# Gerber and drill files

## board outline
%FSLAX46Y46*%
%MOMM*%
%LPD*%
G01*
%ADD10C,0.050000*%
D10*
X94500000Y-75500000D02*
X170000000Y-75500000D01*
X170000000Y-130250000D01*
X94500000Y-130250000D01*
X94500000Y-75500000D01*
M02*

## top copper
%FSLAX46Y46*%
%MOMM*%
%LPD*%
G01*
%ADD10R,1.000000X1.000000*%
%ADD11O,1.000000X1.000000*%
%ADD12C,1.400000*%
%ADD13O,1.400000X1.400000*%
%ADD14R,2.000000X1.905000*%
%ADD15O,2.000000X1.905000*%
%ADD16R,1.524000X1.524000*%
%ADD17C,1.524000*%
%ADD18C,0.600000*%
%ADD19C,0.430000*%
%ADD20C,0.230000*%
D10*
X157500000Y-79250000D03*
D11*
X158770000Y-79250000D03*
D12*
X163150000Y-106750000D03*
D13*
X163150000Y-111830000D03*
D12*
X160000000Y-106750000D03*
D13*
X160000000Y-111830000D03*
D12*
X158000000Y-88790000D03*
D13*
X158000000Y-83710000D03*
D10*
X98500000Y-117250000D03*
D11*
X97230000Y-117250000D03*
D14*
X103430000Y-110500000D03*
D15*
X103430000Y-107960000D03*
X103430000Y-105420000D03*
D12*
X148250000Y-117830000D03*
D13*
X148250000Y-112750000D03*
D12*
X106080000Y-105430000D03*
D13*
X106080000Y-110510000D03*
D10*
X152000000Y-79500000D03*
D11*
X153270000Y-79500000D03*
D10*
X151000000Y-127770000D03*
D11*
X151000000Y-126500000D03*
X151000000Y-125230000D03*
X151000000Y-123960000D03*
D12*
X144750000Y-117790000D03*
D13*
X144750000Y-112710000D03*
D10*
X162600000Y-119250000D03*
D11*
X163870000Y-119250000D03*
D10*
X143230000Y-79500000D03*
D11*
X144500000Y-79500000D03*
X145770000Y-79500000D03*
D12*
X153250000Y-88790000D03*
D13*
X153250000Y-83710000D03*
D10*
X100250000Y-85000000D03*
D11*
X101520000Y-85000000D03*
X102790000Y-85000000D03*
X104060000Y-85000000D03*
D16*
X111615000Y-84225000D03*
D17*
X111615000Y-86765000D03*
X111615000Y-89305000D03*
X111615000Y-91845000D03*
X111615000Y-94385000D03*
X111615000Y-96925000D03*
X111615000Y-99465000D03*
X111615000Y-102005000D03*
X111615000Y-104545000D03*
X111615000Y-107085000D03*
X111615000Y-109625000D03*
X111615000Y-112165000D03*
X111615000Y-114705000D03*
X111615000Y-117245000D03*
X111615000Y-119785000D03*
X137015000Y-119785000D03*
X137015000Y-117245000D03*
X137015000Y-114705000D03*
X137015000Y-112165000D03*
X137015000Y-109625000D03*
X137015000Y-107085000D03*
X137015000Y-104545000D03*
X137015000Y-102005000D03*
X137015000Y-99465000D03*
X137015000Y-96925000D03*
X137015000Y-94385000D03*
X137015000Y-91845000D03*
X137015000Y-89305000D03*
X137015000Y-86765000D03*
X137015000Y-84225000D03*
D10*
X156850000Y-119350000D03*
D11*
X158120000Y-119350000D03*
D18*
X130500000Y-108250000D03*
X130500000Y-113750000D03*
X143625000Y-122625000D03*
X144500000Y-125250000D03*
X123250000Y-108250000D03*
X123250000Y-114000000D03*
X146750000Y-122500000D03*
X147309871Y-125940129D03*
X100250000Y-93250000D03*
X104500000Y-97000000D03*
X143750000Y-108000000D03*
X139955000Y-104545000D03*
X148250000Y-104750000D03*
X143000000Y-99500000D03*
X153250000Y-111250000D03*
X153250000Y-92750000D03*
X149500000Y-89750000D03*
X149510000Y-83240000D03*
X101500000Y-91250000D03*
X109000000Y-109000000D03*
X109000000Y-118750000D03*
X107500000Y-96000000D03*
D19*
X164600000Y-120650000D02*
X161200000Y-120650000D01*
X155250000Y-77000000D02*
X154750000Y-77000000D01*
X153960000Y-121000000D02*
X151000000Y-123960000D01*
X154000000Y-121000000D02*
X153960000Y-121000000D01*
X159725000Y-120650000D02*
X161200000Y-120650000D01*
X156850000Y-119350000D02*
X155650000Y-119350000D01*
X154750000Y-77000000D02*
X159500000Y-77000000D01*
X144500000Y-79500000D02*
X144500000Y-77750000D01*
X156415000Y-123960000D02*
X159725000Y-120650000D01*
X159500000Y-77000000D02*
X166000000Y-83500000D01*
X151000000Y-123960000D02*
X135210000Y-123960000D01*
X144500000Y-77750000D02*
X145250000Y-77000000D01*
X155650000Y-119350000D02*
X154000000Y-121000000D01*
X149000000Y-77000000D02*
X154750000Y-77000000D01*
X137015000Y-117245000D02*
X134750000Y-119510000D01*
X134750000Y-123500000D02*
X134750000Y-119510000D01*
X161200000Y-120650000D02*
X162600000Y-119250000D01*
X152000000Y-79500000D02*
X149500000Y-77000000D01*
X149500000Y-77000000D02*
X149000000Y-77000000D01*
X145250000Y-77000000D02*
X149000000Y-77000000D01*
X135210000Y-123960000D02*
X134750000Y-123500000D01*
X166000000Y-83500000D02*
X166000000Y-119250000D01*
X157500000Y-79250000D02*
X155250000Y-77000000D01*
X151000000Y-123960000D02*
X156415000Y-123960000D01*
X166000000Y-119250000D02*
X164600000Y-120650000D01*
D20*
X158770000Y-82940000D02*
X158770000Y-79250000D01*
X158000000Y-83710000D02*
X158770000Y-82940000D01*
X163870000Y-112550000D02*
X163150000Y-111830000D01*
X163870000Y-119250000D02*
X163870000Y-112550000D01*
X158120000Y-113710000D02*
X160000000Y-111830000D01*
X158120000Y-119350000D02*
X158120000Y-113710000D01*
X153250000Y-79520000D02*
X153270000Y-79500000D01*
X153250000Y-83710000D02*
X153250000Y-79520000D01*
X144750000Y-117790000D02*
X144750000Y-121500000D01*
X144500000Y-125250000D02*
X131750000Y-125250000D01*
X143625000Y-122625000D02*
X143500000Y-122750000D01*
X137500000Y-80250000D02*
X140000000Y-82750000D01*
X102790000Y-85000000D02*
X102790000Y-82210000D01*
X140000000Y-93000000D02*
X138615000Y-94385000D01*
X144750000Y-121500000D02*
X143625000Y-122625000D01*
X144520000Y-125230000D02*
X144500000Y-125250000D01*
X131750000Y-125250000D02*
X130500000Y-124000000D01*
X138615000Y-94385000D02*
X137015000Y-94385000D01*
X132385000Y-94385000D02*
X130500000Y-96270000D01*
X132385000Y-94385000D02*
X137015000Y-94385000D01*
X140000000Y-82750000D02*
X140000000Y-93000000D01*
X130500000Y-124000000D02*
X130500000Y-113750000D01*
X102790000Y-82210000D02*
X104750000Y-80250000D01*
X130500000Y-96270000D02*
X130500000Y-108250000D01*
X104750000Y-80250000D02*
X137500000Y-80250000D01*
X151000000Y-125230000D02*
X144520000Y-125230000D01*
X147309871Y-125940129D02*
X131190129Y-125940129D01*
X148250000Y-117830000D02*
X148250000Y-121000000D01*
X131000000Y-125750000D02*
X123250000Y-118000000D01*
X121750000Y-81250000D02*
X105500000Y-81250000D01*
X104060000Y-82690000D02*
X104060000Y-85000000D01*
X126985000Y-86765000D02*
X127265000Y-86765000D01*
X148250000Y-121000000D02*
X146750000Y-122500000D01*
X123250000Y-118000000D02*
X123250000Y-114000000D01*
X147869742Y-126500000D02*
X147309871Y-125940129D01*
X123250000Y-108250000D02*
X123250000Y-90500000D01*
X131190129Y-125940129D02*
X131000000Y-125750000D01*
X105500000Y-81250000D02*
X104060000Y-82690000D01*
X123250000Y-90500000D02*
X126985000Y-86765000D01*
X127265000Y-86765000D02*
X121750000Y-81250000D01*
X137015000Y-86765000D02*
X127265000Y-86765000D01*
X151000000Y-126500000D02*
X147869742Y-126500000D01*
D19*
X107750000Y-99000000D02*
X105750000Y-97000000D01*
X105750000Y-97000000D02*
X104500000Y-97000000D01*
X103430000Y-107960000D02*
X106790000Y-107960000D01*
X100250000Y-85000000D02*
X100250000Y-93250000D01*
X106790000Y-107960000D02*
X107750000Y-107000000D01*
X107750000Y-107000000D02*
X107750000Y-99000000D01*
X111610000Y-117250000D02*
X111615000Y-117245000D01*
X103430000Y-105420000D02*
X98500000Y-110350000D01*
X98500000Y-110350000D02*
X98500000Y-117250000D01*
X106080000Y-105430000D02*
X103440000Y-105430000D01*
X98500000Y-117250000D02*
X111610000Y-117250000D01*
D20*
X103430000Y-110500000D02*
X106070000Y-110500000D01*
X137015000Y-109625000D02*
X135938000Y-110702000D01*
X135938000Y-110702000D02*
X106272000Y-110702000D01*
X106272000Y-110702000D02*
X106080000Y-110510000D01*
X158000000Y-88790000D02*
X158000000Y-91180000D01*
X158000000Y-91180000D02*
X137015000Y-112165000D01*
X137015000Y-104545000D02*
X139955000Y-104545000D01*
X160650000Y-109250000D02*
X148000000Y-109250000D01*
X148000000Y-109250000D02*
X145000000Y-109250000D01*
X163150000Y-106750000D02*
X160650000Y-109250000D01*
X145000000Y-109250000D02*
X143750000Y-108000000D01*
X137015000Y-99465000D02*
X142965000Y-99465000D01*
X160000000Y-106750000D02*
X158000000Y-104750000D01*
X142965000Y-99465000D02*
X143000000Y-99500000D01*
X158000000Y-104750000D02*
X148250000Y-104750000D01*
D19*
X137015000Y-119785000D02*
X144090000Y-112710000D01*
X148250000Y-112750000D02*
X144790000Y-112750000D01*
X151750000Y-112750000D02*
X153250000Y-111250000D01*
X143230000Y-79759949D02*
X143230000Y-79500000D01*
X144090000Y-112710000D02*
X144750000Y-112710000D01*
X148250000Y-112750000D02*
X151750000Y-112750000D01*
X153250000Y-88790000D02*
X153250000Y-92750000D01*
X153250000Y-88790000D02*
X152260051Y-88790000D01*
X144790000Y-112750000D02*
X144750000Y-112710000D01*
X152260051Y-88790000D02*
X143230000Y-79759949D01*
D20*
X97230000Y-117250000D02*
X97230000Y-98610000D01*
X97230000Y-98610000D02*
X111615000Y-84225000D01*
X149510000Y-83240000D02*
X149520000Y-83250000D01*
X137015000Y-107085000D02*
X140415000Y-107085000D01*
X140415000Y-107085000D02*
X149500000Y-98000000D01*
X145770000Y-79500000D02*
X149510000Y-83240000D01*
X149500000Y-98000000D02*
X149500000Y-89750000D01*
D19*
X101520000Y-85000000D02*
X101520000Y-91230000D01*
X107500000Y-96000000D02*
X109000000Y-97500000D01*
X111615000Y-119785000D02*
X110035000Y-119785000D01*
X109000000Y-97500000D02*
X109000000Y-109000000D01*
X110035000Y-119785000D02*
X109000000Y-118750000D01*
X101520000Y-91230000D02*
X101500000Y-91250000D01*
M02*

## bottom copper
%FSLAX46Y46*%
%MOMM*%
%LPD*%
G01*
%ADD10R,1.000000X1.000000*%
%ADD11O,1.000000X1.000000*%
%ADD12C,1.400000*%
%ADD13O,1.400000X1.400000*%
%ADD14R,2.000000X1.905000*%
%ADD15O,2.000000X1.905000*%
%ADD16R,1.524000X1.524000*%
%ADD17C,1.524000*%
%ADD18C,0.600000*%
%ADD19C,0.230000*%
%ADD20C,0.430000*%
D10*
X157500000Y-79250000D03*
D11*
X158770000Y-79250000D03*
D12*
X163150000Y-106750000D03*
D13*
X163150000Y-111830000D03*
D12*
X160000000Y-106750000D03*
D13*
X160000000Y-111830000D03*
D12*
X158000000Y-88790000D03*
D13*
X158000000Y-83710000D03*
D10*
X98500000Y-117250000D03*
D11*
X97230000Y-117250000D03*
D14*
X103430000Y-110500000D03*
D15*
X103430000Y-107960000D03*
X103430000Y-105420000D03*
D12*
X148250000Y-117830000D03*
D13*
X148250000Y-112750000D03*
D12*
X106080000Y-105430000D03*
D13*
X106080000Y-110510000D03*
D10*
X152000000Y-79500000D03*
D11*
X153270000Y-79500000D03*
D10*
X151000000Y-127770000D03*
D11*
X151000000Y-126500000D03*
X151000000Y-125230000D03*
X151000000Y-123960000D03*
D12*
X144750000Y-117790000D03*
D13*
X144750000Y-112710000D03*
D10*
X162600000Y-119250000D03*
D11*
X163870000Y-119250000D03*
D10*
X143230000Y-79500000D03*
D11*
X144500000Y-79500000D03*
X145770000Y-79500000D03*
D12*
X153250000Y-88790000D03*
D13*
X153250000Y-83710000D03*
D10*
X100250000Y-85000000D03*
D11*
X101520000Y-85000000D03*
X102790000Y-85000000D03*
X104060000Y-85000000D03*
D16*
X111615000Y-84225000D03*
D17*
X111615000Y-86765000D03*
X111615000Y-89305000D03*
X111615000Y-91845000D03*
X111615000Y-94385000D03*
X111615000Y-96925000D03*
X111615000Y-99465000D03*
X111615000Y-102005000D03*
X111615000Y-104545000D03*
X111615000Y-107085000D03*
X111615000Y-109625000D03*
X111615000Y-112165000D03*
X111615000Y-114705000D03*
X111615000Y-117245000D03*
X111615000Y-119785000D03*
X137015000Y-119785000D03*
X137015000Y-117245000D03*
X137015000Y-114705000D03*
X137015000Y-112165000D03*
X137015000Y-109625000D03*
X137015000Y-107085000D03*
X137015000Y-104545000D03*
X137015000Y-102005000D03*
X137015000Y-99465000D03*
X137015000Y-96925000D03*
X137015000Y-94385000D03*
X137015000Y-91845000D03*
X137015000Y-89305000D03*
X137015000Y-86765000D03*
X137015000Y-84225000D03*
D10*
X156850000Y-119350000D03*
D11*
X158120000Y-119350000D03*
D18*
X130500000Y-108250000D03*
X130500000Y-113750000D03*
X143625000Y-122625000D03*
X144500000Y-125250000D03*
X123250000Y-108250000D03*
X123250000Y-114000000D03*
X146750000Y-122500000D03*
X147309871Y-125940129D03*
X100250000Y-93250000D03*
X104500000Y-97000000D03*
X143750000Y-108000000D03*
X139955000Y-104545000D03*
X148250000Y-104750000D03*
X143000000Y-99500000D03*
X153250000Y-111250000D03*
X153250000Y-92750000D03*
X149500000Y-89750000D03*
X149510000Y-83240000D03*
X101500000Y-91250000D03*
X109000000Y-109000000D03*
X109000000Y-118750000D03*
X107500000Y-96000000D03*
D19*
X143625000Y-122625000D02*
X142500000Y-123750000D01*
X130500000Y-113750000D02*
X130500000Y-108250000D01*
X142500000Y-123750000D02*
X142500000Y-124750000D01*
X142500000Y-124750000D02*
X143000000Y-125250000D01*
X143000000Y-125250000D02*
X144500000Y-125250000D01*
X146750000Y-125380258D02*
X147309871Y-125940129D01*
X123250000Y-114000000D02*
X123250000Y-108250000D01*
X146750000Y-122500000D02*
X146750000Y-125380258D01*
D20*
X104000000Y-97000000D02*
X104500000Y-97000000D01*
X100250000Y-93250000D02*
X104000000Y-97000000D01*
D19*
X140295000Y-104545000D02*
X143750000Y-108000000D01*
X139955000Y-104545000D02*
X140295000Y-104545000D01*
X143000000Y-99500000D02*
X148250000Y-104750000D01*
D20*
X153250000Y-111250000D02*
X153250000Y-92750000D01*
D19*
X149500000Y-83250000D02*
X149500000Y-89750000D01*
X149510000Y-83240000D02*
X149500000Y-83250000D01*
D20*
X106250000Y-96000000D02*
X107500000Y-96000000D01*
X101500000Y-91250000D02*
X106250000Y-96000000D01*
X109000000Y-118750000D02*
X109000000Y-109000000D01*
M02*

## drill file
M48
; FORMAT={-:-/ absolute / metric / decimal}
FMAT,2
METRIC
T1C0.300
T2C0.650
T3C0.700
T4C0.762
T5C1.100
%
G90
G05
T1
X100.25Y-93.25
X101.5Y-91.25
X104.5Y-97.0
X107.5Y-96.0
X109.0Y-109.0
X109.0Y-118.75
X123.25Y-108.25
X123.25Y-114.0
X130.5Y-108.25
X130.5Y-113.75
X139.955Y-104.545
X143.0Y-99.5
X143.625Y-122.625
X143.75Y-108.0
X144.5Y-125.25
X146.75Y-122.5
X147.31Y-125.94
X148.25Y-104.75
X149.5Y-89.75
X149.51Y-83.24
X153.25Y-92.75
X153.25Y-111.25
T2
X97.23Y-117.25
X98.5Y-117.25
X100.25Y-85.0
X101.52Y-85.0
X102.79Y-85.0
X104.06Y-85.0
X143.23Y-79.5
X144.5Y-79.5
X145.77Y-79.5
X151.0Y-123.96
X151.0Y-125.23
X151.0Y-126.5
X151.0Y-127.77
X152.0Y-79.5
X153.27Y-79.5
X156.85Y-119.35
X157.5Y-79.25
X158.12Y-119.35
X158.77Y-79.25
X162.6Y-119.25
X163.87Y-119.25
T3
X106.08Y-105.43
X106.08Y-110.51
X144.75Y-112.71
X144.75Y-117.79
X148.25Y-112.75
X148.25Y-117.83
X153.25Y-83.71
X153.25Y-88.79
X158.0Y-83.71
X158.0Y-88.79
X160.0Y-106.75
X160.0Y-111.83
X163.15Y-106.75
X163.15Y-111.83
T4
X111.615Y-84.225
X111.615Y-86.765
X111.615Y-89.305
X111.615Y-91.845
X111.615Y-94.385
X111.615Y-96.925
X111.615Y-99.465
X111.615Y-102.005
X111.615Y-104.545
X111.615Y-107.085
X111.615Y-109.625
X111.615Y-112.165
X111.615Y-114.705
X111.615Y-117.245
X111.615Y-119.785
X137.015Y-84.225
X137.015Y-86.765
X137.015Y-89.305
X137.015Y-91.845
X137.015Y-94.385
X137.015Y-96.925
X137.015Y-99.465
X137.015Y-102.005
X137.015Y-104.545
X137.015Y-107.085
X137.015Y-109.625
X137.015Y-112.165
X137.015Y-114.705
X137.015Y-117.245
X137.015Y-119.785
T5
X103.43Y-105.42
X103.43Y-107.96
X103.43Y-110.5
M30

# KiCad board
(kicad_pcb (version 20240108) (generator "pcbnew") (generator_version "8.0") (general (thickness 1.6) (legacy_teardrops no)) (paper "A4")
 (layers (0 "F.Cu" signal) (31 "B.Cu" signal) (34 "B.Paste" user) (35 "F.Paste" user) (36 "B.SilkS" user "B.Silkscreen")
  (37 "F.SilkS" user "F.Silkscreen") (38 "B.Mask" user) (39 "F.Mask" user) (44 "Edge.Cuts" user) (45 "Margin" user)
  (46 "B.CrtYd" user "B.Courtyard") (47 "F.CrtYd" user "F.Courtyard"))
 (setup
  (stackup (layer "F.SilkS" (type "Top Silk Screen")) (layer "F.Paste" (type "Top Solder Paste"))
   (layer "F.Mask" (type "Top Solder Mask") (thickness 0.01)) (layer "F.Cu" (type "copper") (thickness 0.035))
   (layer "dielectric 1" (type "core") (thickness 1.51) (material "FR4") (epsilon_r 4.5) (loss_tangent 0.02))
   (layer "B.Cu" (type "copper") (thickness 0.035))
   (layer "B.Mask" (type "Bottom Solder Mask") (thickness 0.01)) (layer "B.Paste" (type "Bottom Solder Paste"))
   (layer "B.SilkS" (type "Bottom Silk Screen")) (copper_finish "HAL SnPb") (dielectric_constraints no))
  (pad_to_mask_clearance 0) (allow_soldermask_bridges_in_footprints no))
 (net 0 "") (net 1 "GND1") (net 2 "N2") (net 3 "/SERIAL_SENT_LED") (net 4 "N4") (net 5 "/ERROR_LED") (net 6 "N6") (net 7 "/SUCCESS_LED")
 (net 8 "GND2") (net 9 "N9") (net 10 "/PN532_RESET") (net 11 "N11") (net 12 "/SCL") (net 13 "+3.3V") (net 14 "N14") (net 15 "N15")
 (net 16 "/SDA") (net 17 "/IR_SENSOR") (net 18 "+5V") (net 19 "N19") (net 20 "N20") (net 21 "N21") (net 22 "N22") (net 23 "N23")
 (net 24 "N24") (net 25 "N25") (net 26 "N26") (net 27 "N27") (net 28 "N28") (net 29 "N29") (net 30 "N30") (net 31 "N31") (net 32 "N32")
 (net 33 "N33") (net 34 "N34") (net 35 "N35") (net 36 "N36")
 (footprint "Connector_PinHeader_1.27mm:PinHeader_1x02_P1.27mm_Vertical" (layer "F.Cu") (at 157.5 79.25 90)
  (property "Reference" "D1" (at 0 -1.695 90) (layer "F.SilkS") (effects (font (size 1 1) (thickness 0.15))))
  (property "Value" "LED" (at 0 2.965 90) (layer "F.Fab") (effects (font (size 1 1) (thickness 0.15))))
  (pad "1" thru_hole rect (at 0 0 90) (size 1 1) (drill 0.65) (layers "*.Cu" "*.Mask") (remove_unused_layers no) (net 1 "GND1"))
  (pad "2" thru_hole oval (at 0 1.27 90) (size 1 1) (drill 0.65) (layers "*.Cu" "*.Mask") (remove_unused_layers no) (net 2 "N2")))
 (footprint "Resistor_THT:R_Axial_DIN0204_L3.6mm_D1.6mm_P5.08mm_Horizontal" (layer "F.Cu") (at 163.15 106.75 -90)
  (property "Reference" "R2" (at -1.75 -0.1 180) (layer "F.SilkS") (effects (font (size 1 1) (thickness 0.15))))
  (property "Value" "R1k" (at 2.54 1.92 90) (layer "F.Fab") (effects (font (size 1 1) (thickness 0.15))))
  (pad "1" thru_hole circle (at 0 0 270) (size 1.4 1.4) (drill 0.7) (layers "*.Cu" "*.Mask") (remove_unused_layers no)
   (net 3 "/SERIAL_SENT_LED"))
  (pad "2" thru_hole oval (at 5.08 0 270) (size 1.4 1.4) (drill 0.7) (layers "*.Cu" "*.Mask") (remove_unused_layers no) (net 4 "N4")))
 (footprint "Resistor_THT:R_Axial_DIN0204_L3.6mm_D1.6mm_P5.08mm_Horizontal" (layer "F.Cu") (at 160 106.75 -90)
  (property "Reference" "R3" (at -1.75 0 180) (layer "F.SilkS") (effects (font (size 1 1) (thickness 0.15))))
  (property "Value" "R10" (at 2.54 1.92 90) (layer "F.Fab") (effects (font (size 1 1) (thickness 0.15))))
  (pad "1" thru_hole circle (at 0 0 270) (size 1.4 1.4) (drill 0.7) (layers "*.Cu" "*.Mask") (remove_unused_layers no) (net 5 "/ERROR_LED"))
  (pad "2" thru_hole oval (at 5.08 0 270) (size 1.4 1.4) (drill 0.7) (layers "*.Cu" "*.Mask") (remove_unused_layers no) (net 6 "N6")))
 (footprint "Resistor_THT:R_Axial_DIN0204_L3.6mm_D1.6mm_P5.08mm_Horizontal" (layer "F.Cu") (at 158 88.79 90)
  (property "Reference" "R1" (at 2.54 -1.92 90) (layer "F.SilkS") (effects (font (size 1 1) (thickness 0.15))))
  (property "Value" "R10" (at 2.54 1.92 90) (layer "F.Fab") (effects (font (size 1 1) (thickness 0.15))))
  (pad "1" thru_hole circle (at 0 0 90) (size 1.4 1.4) (drill 0.7) (layers "*.Cu" "*.Mask") (remove_unused_layers no) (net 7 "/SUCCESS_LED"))
  (pad "2" thru_hole oval (at 5.08 0 90) (size 1.4 1.4) (drill 0.7) (layers "*.Cu" "*.Mask") (remove_unused_layers no) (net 2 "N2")))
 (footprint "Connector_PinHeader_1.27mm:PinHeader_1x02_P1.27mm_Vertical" (layer "F.Cu") (at 98.5 117.25 -90)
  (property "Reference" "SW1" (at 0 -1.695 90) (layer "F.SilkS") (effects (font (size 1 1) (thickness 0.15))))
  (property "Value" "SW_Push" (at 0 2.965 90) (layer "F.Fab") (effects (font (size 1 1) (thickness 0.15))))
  (pad "1" thru_hole rect (at 0 0 270) (size 1 1) (drill 0.65) (layers "*.Cu" "*.Mask") (remove_unused_layers no) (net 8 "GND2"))
  (pad "2" thru_hole oval (at 0 1.27 270) (size 1 1) (drill 0.65) (layers "*.Cu" "*.Mask") (remove_unused_layers no) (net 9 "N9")))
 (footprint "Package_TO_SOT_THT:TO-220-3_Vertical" (layer "F.Cu") (at 103.43 110.5 90)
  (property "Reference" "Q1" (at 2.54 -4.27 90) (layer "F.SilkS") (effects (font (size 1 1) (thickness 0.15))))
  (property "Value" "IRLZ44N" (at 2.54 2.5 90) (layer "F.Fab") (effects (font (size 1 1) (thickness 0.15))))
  (pad "1" thru_hole rect (at 0 0 90) (size 1.905 2) (drill 1.1) (layers "*.Cu" "*.Mask") (remove_unused_layers no) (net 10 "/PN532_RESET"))
  (pad "2" thru_hole oval (at 2.54 0 90) (size 1.905 2) (drill 1.1) (layers "*.Cu" "*.Mask") (remove_unused_layers no) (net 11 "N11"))
  (pad "3" thru_hole oval (at 5.08 0 90) (size 1.905 2) (drill 1.1) (layers "*.Cu" "*.Mask") (remove_unused_layers no) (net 8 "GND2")))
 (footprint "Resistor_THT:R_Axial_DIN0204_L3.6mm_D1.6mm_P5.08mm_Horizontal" (layer "F.Cu") (at 148.25 117.83 90)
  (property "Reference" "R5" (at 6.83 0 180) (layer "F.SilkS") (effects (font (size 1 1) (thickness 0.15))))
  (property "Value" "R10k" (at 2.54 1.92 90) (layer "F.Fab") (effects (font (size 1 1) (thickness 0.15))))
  (pad "1" thru_hole circle (at 0 0 90) (size 1.4 1.4) (drill 0.7) (layers "*.Cu" "*.Mask") (remove_unused_layers no) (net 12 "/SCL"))
  (pad "2" thru_hole oval (at 5.08 0 90) (size 1.4 1.4) (drill 0.7) (layers "*.Cu" "*.Mask") (remove_unused_layers no) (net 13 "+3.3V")))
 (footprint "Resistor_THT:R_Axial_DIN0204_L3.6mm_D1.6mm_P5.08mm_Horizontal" (layer "F.Cu") (at 106.08 105.43 -90)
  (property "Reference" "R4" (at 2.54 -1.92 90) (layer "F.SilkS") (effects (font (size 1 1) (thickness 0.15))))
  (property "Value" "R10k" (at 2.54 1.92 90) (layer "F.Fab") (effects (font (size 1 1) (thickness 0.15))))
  (pad "1" thru_hole circle (at 0 0 270) (size 1.4 1.4) (drill 0.7) (layers "*.Cu" "*.Mask") (remove_unused_layers no) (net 8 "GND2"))
  (pad "2" thru_hole oval (at 5.08 0 270) (size 1.4 1.4) (drill 0.7) (layers "*.Cu" "*.Mask") (remove_unused_layers no)
   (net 10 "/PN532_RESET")))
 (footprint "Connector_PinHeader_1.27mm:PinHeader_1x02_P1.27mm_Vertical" (layer "F.Cu") (at 152 79.5 90)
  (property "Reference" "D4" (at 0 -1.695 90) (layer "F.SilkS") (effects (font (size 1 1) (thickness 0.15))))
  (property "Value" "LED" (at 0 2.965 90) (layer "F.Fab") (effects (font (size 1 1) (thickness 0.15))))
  (pad "1" thru_hole rect (at 0 0 90) (size 1 1) (drill 0.65) (layers "*.Cu" "*.Mask") (remove_unused_layers no) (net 1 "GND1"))
  (pad "2" thru_hole oval (at 0 1.27 90) (size 1 1) (drill 0.65) (layers "*.Cu" "*.Mask") (remove_unused_layers no) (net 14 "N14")))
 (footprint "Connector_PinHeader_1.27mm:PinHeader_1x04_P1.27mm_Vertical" (layer "F.Cu") (at 151 127.77 180)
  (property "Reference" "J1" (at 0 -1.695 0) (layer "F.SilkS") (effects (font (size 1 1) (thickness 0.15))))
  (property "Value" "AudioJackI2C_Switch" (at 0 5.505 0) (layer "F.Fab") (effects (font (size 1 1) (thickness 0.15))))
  (pad "1" thru_hole rect (at 0 0 180) (size 1 1) (drill 0.65) (layers "*.Cu" "*.Mask") (remove_unused_layers no) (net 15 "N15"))
  (pad "2" thru_hole oval (at 0 1.27 180) (size 1 1) (drill 0.65) (layers "*.Cu" "*.Mask") (remove_unused_layers no) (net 12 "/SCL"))
  (pad "3" thru_hole oval (at 0 2.54 180) (size 1 1) (drill 0.65) (layers "*.Cu" "*.Mask") (remove_unused_layers no) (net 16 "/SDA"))
  (pad "4" thru_hole oval (at 0 3.81 180) (size 1 1) (drill 0.65) (layers "*.Cu" "*.Mask") (remove_unused_layers no) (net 1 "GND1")))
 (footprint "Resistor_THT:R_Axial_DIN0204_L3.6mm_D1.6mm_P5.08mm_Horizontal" (layer "F.Cu") (at 144.75 117.79 90)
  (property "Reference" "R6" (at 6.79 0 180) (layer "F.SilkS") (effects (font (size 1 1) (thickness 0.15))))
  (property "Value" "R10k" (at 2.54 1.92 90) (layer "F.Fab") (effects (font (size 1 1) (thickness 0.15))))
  (pad "1" thru_hole circle (at 0 0 90) (size 1.4 1.4) (drill 0.7) (layers "*.Cu" "*.Mask") (remove_unused_layers no) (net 16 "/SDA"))
  (pad "2" thru_hole oval (at 5.08 0 90) (size 1.4 1.4) (drill 0.7) (layers "*.Cu" "*.Mask") (remove_unused_layers no) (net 13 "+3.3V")))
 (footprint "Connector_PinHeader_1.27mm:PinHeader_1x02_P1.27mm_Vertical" (layer "F.Cu") (at 162.6 119.25 90)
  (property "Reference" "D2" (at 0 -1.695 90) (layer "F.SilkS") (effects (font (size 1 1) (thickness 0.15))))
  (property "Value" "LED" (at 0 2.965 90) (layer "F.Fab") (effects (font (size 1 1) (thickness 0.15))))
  (pad "1" thru_hole rect (at 0 0 90) (size 1 1) (drill 0.65) (layers "*.Cu" "*.Mask") (remove_unused_layers no) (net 1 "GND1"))
  (pad "2" thru_hole oval (at 0 1.27 90) (size 1 1) (drill 0.65) (layers "*.Cu" "*.Mask") (remove_unused_layers no) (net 4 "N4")))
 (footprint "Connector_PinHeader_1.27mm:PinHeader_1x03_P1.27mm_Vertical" (layer "F.Cu") (at 143.23 79.5 90)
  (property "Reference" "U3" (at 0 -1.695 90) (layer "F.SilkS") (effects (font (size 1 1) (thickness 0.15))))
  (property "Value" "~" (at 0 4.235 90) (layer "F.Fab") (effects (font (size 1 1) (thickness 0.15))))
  (pad "1" thru_hole rect (at 0 0 90) (size 1 1) (drill 0.65) (layers "*.Cu" "*.Mask") (remove_unused_layers no) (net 13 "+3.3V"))
  (pad "2" thru_hole oval (at 0 1.27 90) (size 1 1) (drill 0.65) (layers "*.Cu" "*.Mask") (remove_unused_layers no) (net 1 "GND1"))
  (pad "3" thru_hole oval (at 0 2.54 90) (size 1 1) (drill 0.65) (layers "*.Cu" "*.Mask") (remove_unused_layers no) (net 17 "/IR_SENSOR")))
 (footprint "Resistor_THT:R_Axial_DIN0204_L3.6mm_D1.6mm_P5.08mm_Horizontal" (layer "F.Cu") (at 153.25 88.79 90)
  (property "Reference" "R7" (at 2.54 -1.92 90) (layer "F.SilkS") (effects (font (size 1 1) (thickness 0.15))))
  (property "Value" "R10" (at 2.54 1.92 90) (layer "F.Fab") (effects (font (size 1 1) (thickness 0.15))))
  (pad "1" thru_hole circle (at 0 0 90) (size 1.4 1.4) (drill 0.7) (layers "*.Cu" "*.Mask") (remove_unused_layers no) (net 13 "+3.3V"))
  (pad "2" thru_hole oval (at 5.08 0 90) (size 1.4 1.4) (drill 0.7) (layers "*.Cu" "*.Mask") (remove_unused_layers no) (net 14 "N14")))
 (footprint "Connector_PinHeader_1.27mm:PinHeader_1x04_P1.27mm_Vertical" (layer "F.Cu") (at 100.25 85 90)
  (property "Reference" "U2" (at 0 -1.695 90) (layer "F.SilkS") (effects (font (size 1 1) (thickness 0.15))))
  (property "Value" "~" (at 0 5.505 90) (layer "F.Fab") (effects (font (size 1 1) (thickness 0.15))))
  (pad "1" thru_hole rect (at 0 0 90) (size 1 1) (drill 0.65) (layers "*.Cu" "*.Mask") (remove_unused_layers no) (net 11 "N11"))
  (pad "2" thru_hole oval (at 0 1.27 90) (size 1 1) (drill 0.65) (layers "*.Cu" "*.Mask") (remove_unused_layers no) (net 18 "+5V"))
  (pad "3" thru_hole oval (at 0 2.54 90) (size 1 1) (drill 0.65) (layers "*.Cu" "*.Mask") (remove_unused_layers no) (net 16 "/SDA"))
  (pad "4" thru_hole oval (at 0 3.81 90) (size 1 1) (drill 0.65) (layers "*.Cu" "*.Mask") (remove_unused_layers no) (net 12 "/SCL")))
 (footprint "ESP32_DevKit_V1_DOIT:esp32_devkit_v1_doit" (layer "F.Cu") (at 124.315 84.225)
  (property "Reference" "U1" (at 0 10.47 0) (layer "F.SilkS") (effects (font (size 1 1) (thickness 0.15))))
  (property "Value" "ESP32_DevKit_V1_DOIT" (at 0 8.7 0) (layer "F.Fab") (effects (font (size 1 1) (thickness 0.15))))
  (pad "1" thru_hole rect (at -12.7 0) (size 1.524 1.524) (drill 0.762) (layers "*.Cu" "*.Mask") (remove_unused_layers no) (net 9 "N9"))
  (pad "2" thru_hole circle (at -12.7 2.54) (size 1.524 1.524) (drill 0.762) (layers "*.Cu" "*.Mask") (remove_unused_layers no)
   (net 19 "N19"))
  (pad "3" thru_hole circle (at -12.7 5.08) (size 1.524 1.524) (drill 0.762) (layers "*.Cu" "*.Mask") (remove_unused_layers no)
   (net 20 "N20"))
  (pad "4" thru_hole circle (at -12.7 7.62) (size 1.524 1.524) (drill 0.762) (layers "*.Cu" "*.Mask") (remove_unused_layers no)
   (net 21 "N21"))
  (pad "5" thru_hole circle (at -12.7 10.16) (size 1.524 1.524) (drill 0.762) (layers "*.Cu" "*.Mask") (remove_unused_layers no)
   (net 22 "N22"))
  (pad "6" thru_hole circle (at -12.7 12.7) (size 1.524 1.524) (drill 0.762) (layers "*.Cu" "*.Mask") (remove_unused_layers no)
   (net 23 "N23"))
  (pad "7" thru_hole circle (at -12.7 15.24) (size 1.524 1.524) (drill 0.762) (layers "*.Cu" "*.Mask") (remove_unused_layers no)
   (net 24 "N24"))
  (pad "8" thru_hole circle (at -12.7 17.78) (size 1.524 1.524) (drill 0.762) (layers "*.Cu" "*.Mask") (remove_unused_layers no)
   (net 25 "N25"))
  (pad "9" thru_hole circle (at -12.7 20.32) (size 1.524 1.524) (drill 0.762) (layers "*.Cu" "*.Mask") (remove_unused_layers no)
   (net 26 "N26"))
  (pad "10" thru_hole circle (at -12.7 22.86) (size 1.524 1.524) (drill 0.762) (layers "*.Cu" "*.Mask") (remove_unused_layers no)
   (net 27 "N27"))
  (pad "11" thru_hole circle (at -12.7 25.4) (size 1.524 1.524) (drill 0.762) (layers "*.Cu" "*.Mask") (remove_unused_layers no)
   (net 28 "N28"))
  (pad "12" thru_hole circle (at -12.7 27.94) (size 1.524 1.524) (drill 0.762) (layers "*.Cu" "*.Mask") (remove_unused_layers no)
   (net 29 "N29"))
  (pad "13" thru_hole circle (at -12.7 30.48) (size 1.524 1.524) (drill 0.762) (layers "*.Cu" "*.Mask") (remove_unused_layers no)
   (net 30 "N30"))
  (pad "14" thru_hole circle (at -12.7 33.02) (size 1.524 1.524) (drill 0.762) (layers "*.Cu" "*.Mask") (remove_unused_layers no)
   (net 8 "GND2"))
  (pad "15" thru_hole circle (at -12.7 35.56) (size 1.524 1.524) (drill 0.762) (layers "*.Cu" "*.Mask") (remove_unused_layers no)
   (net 18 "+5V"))
  (pad "16" thru_hole circle (at 12.7 35.56) (size 1.524 1.524) (drill 0.762) (layers "*.Cu" "*.Mask") (remove_unused_layers no)
   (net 13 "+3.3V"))
  (pad "17" thru_hole circle (at 12.7 33.02) (size 1.524 1.524) (drill 0.762) (layers "*.Cu" "*.Mask") (remove_unused_layers no)
   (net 1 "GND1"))
  (pad "18" thru_hole circle (at 12.7 30.48) (size 1.524 1.524) (drill 0.762) (layers "*.Cu" "*.Mask") (remove_unused_layers no)
   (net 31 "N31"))
  (pad "19" thru_hole circle (at 12.7 27.94) (size 1.524 1.524) (drill 0.762) (layers "*.Cu" "*.Mask") (remove_unused_layers no)
   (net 7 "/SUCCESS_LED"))
  (pad "20" thru_hole circle (at 12.7 25.4) (size 1.524 1.524) (drill 0.762) (layers "*.Cu" "*.Mask") (remove_unused_layers no)
   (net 10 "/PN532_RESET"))
  (pad "21" thru_hole circle (at 12.7 22.86) (size 1.524 1.524) (drill 0.762) (layers "*.Cu" "*.Mask") (remove_unused_layers no)
   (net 17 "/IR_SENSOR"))
  (pad "22" thru_hole circle (at 12.7 20.32) (size 1.524 1.524) (drill 0.762) (layers "*.Cu" "*.Mask") (remove_unused_layers no)
   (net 3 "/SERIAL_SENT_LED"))
  (pad "23" thru_hole circle (at 12.7 17.78) (size 1.524 1.524) (drill 0.762) (layers "*.Cu" "*.Mask") (remove_unused_layers no)
   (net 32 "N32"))
  (pad "24" thru_hole circle (at 12.7 15.24) (size 1.524 1.524) (drill 0.762) (layers "*.Cu" "*.Mask") (remove_unused_layers no)
   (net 5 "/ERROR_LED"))
  (pad "25" thru_hole circle (at 12.7 12.7) (size 1.524 1.524) (drill 0.762) (layers "*.Cu" "*.Mask") (remove_unused_layers no)
   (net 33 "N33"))
  (pad "26" thru_hole circle (at 12.7 10.16) (size 1.524 1.524) (drill 0.762) (layers "*.Cu" "*.Mask") (remove_unused_layers no)
   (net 16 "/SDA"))
  (pad "27" thru_hole circle (at 12.7 7.62) (size 1.524 1.524) (drill 0.762) (layers "*.Cu" "*.Mask") (remove_unused_layers no)
   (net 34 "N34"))
  (pad "28" thru_hole circle (at 12.7 5.08) (size 1.524 1.524) (drill 0.762) (layers "*.Cu" "*.Mask") (remove_unused_layers no)
   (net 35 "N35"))
  (pad "29" thru_hole circle (at 12.7 2.54) (size 1.524 1.524) (drill 0.762) (layers "*.Cu" "*.Mask") (remove_unused_layers no)
   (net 12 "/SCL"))
  (pad "30" thru_hole circle (at 12.7 0) (size 1.524 1.524) (drill 0.762) (layers "*.Cu" "*.Mask") (remove_unused_layers no) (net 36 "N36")))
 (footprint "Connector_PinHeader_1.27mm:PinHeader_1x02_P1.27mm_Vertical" (layer "F.Cu") (at 156.85 119.35 90)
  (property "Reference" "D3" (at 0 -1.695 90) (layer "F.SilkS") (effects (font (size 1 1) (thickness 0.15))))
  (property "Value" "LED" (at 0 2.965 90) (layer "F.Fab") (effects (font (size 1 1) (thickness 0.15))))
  (pad "1" thru_hole rect (at 0 0 90) (size 1 1) (drill 0.65) (layers "*.Cu" "*.Mask") (remove_unused_layers no) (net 1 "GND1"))
  (pad "2" thru_hole oval (at 0 1.27 90) (size 1 1) (drill 0.65) (layers "*.Cu" "*.Mask") (remove_unused_layers no) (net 6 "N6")))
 (gr_rect (start 94.5 75.5) (end 170 130.25) (locked yes) (stroke (width 0.05) (type default)) (fill none) (layer "Edge.Cuts"))
 (segment (start 164.6 120.65) (end 161.2 120.65) (width 0.43) (layer "F.Cu") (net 1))
 (segment (start 155.25 77) (end 154.75 77) (width 0.43) (layer "F.Cu") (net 1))
 (segment (start 153.96 121) (end 151 123.96) (width 0.43) (layer "F.Cu") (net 1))
 (segment (start 154 121) (end 153.96 121) (width 0.43) (layer "F.Cu") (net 1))
 (segment (start 159.725 120.65) (end 161.2 120.65) (width 0.43) (layer "F.Cu") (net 1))
 (segment (start 156.85 119.35) (end 155.65 119.35) (width 0.43) (layer "F.Cu") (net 1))
 (segment (start 154.75 77) (end 159.5 77) (width 0.43) (layer "F.Cu") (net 1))
 (segment (start 144.5 79.5) (end 144.5 77.75) (width 0.43) (layer "F.Cu") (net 1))
 (segment (start 156.415 123.96) (end 159.725 120.65) (width 0.43) (layer "F.Cu") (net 1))
 (segment (start 159.5 77) (end 166 83.5) (width 0.43) (layer "F.Cu") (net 1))
 (segment (start 151 123.96) (end 135.21 123.96) (width 0.43) (layer "F.Cu") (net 1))
 (segment (start 144.5 77.75) (end 145.25 77) (width 0.43) (layer "F.Cu") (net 1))
 (segment (start 155.65 119.35) (end 154 121) (width 0.43) (layer "F.Cu") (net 1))
 (segment (start 149 77) (end 154.75 77) (width 0.43) (layer "F.Cu") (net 1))
 (segment (start 137.015 117.245) (end 134.75 119.51) (width 0.43) (layer "F.Cu") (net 1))
 (segment (start 134.75 123.5) (end 134.75 119.51) (width 0.43) (layer "F.Cu") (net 1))
 (segment (start 161.2 120.65) (end 162.6 119.25) (width 0.43) (layer "F.Cu") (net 1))
 (segment (start 152 79.5) (end 149.5 77) (width 0.43) (layer "F.Cu") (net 1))
 (segment (start 149.5 77) (end 149 77) (width 0.43) (layer "F.Cu") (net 1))
 (segment (start 145.25 77) (end 149 77) (width 0.43) (layer "F.Cu") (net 1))
 (segment (start 135.21 123.96) (end 134.75 123.5) (width 0.43) (layer "F.Cu") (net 1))
 (segment (start 166 83.5) (end 166 119.25) (width 0.43) (layer "F.Cu") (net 1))
 (segment (start 157.5 79.25) (end 155.25 77) (width 0.43) (layer "F.Cu") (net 1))
 (segment (start 151 123.96) (end 156.415 123.96) (width 0.43) (layer "F.Cu") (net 1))
 (segment (start 166 119.25) (end 164.6 120.65) (width 0.43) (layer "F.Cu") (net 1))
 (segment (start 158.77 82.94) (end 158.77 79.25) (width 0.23) (layer "F.Cu") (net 2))
 (segment (start 158 83.71) (end 158.77 82.94) (width 0.23) (layer "F.Cu") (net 2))
 (segment (start 163.87 112.55) (end 163.15 111.83) (width 0.23) (layer "F.Cu") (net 4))
 (segment (start 163.87 119.25) (end 163.87 112.55) (width 0.23) (layer "F.Cu") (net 4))
 (segment (start 158.12 113.71) (end 160 111.83) (width 0.23) (layer "F.Cu") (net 6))
 (segment (start 158.12 119.35) (end 158.12 113.71) (width 0.23) (layer "F.Cu") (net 6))
 (segment (start 153.25 79.52) (end 153.27 79.5) (width 0.23) (layer "F.Cu") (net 14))
 (segment (start 153.25 83.71) (end 153.25 79.52) (width 0.23) (layer "F.Cu") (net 14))
 (segment (start 144.75 117.79) (end 144.75 121.5) (width 0.23) (layer "F.Cu") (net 16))
 (segment (start 144.5 125.25) (end 131.75 125.25) (width 0.23) (layer "F.Cu") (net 16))
 (segment (start 143.625 122.625) (end 143.5 122.75) (width 0.23) (layer "F.Cu") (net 16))
 (segment (start 137.5 80.25) (end 140 82.75) (width 0.23) (layer "F.Cu") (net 16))
 (segment (start 102.79 85) (end 102.79 82.21) (width 0.23) (layer "F.Cu") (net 16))
 (segment (start 140 93) (end 138.615 94.385) (width 0.23) (layer "F.Cu") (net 16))
 (segment (start 144.75 121.5) (end 143.625 122.625) (width 0.23) (layer "F.Cu") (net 16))
 (segment (start 144.52 125.23) (end 144.5 125.25) (width 0.23) (layer "F.Cu") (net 16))
 (segment (start 131.75 125.25) (end 130.5 124) (width 0.23) (layer "F.Cu") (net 16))
 (segment (start 138.615 94.385) (end 137.015 94.385) (width 0.23) (layer "F.Cu") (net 16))
 (segment (start 132.385 94.385) (end 130.5 96.27) (width 0.23) (layer "F.Cu") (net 16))
 (segment (start 132.385 94.385) (end 137.015 94.385) (width 0.23) (layer "F.Cu") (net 16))
 (segment (start 140 82.75) (end 140 93) (width 0.23) (layer "F.Cu") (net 16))
 (segment (start 130.5 124) (end 130.5 113.75) (width 0.23) (layer "F.Cu") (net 16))
 (segment (start 102.79 82.21) (end 104.75 80.25) (width 0.23) (layer "F.Cu") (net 16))
 (segment (start 130.5 96.27) (end 130.5 108.25) (width 0.23) (layer "F.Cu") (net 16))
 (segment (start 104.75 80.25) (end 137.5 80.25) (width 0.23) (layer "F.Cu") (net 16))
 (segment (start 151 125.23) (end 144.52 125.23) (width 0.23) (layer "F.Cu") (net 16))
 (via (at 130.5 108.25) (size 0.6) (drill 0.3) (layers "F.Cu" "B.Cu") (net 16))
 (via (at 130.5 113.75) (size 0.6) (drill 0.3) (layers "F.Cu" "B.Cu") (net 16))
 (via (at 143.625 122.625) (size 0.6) (drill 0.3) (layers "F.Cu" "B.Cu") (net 16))
 (via (at 144.5 125.25) (size 0.6) (drill 0.3) (layers "F.Cu" "B.Cu") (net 16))
 (segment (start 143.625 122.625) (end 142.5 123.75) (width 0.23) (layer "B.Cu") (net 16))
 (segment (start 130.5 113.75) (end 130.5 108.25) (width 0.23) (layer "B.Cu") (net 16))
 (segment (start 142.5 123.75) (end 142.5 124.75) (width 0.23) (layer "B.Cu") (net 16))
 (segment (start 142.5 124.75) (end 143 125.25) (width 0.23) (layer "B.Cu") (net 16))
 (segment (start 143 125.25) (end 144.5 125.25) (width 0.23) (layer "B.Cu") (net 16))
 (segment (start 147.309871 125.940129) (end 131.190129 125.940129) (width 0.23) (layer "F.Cu") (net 12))
 (segment (start 148.25 117.83) (end 148.25 121) (width 0.23) (layer "F.Cu") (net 12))
 (segment (start 131 125.75) (end 123.25 118) (width 0.23) (layer "F.Cu") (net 12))
 (segment (start 121.75 81.25) (end 105.5 81.25) (width 0.23) (layer "F.Cu") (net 12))
 (segment (start 104.06 82.69) (end 104.06 85) (width 0.23) (layer "F.Cu") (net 12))
 (segment (start 126.985 86.765) (end 127.265 86.765) (width 0.23) (layer "F.Cu") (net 12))
 (segment (start 148.25 121) (end 146.75 122.5) (width 0.23) (layer "F.Cu") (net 12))
 (segment (start 123.25 118) (end 123.25 114) (width 0.23) (layer "F.Cu") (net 12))
 (segment (start 147.869742 126.5) (end 147.309871 125.940129) (width 0.23) (layer "F.Cu") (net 12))
 (segment (start 123.25 108.25) (end 123.25 90.5) (width 0.23) (layer "F.Cu") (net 12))
 (segment (start 131.190129 125.940129) (end 131 125.75) (width 0.23) (layer "F.Cu") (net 12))
 (segment (start 105.5 81.25) (end 104.06 82.69) (width 0.23) (layer "F.Cu") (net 12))
 (segment (start 123.25 90.5) (end 126.985 86.765) (width 0.23) (layer "F.Cu") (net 12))
 (segment (start 127.265 86.765) (end 121.75 81.25) (width 0.23) (layer "F.Cu") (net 12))
 (segment (start 137.015 86.765) (end 127.265 86.765) (width 0.23) (layer "F.Cu") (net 12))
 (segment (start 151 126.5) (end 147.869742 126.5) (width 0.23) (layer "F.Cu") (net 12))
 (via (at 123.25 108.25) (size 0.6) (drill 0.3) (layers "F.Cu" "B.Cu") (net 12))
 (via (at 123.25 114) (size 0.6) (drill 0.3) (layers "F.Cu" "B.Cu") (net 12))
 (via (at 146.75 122.5) (size 0.6) (drill 0.3) (layers "F.Cu" "B.Cu") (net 12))
 (via (at 147.309871 125.940129) (size 0.6) (drill 0.3) (layers "F.Cu" "B.Cu") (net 12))
 (segment (start 146.75 125.380258) (end 147.309871 125.940129) (width 0.23) (layer "B.Cu") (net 12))
 (segment (start 123.25 114) (end 123.25 108.25) (width 0.23) (layer "B.Cu") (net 12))
 (segment (start 146.75 122.5) (end 146.75 125.380258) (width 0.23) (layer "B.Cu") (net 12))
 (segment (start 107.75 99) (end 105.75 97) (width 0.43) (layer "F.Cu") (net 11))
 (segment (start 105.75 97) (end 104.5 97) (width 0.43) (layer "F.Cu") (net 11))
 (segment (start 103.43 107.96) (end 106.79 107.96) (width 0.43) (layer "F.Cu") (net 11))
 (segment (start 100.25 85) (end 100.25 93.25) (width 0.43) (layer "F.Cu") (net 11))
 (segment (start 106.79 107.96) (end 107.75 107) (width 0.43) (layer "F.Cu") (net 11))
 (segment (start 107.75 107) (end 107.75 99) (width 0.43) (layer "F.Cu") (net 11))
 (via (at 100.25 93.25) (size 0.6) (drill 0.3) (layers "F.Cu" "B.Cu") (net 11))
 (via (at 104.5 97) (size 0.6) (drill 0.3) (layers "F.Cu" "B.Cu") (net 11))
 (segment (start 104 97) (end 104.5 97) (width 0.43) (layer "B.Cu") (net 11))
 (segment (start 100.25 93.25) (end 104 97) (width 0.43) (layer "B.Cu") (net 11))
 (segment (start 111.61 117.25) (end 111.615 117.245) (width 0.43) (layer "F.Cu") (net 8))
 (segment (start 103.43 105.42) (end 98.5 110.35) (width 0.43) (layer "F.Cu") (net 8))
 (segment (start 98.5 110.35) (end 98.5 117.25) (width 0.43) (layer "F.Cu") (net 8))
 (segment (start 106.08 105.43) (end 103.44 105.43) (width 0.43) (layer "F.Cu") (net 8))
 (segment (start 98.5 117.25) (end 111.61 117.25) (width 0.43) (layer "F.Cu") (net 8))
 (segment (start 103.43 110.5) (end 106.07 110.5) (width 0.23) (layer "F.Cu") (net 10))
 (segment (start 137.015 109.625) (end 135.938 110.702) (width 0.23) (layer "F.Cu") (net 10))
 (segment (start 135.938 110.702) (end 106.272 110.702) (width 0.23) (layer "F.Cu") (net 10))
 (segment (start 106.272 110.702) (end 106.08 110.51) (width 0.23) (layer "F.Cu") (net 10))
 (segment (start 158 88.79) (end 158 91.18) (width 0.23) (layer "F.Cu") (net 7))
 (segment (start 158 91.18) (end 137.015 112.165) (width 0.23) (layer "F.Cu") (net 7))
 (segment (start 137.015 104.545) (end 139.955 104.545) (width 0.23) (layer "F.Cu") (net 3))
 (segment (start 160.65 109.25) (end 148 109.25) (width 0.23) (layer "F.Cu") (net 3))
 (segment (start 148 109.25) (end 145 109.25) (width 0.23) (layer "F.Cu") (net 3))
 (segment (start 163.15 106.75) (end 160.65 109.25) (width 0.23) (layer "F.Cu") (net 3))
 (segment (start 145 109.25) (end 143.75 108) (width 0.23) (layer "F.Cu") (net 3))
 (via (at 143.75 108) (size 0.6) (drill 0.3) (layers "F.Cu" "B.Cu") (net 3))
 (via (at 139.955 104.545) (size 0.6) (drill 0.3) (layers "F.Cu" "B.Cu") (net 3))
 (segment (start 140.295 104.545) (end 143.75 108) (width 0.23) (layer "B.Cu") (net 3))
 (segment (start 139.955 104.545) (end 140.295 104.545) (width 0.23) (layer "B.Cu") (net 3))
 (segment (start 137.015 99.465) (end 142.965 99.465) (width 0.23) (layer "F.Cu") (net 5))
 (segment (start 160 106.75) (end 158 104.75) (width 0.23) (layer "F.Cu") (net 5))
 (segment (start 142.965 99.465) (end 143 99.5) (width 0.23) (layer "F.Cu") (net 5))
 (segment (start 158 104.75) (end 148.25 104.75) (width 0.23) (layer "F.Cu") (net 5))
 (via (at 148.25 104.75) (size 0.6) (drill 0.3) (layers "F.Cu" "B.Cu") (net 5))
 (via (at 143 99.5) (size 0.6) (drill 0.3) (layers "F.Cu" "B.Cu") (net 5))
 (segment (start 143 99.5) (end 148.25 104.75) (width 0.23) (layer "B.Cu") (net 5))
 (segment (start 137.015 119.785) (end 144.09 112.71) (width 0.43) (layer "F.Cu") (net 13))
 (segment (start 148.25 112.75) (end 144.79 112.75) (width 0.43) (layer "F.Cu") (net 13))
 (segment (start 151.75 112.75) (end 153.25 111.25) (width 0.43) (layer "F.Cu") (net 13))
 (segment (start 143.23 79.759949) (end 143.23 79.5) (width 0.43) (layer "F.Cu") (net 13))
 (segment (start 144.09 112.71) (end 144.75 112.71) (width 0.43) (layer "F.Cu") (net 13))
 (segment (start 148.25 112.75) (end 151.75 112.75) (width 0.43) (layer "F.Cu") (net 13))
 (segment (start 153.25 88.79) (end 153.25 92.75) (width 0.43) (layer "F.Cu") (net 13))
 (segment (start 153.25 88.79) (end 152.260051 88.79) (width 0.43) (layer "F.Cu") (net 13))
 (segment (start 144.79 112.75) (end 144.75 112.71) (width 0.43) (layer "F.Cu") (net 13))
 (segment (start 152.260051 88.79) (end 143.23 79.759949) (width 0.43) (layer "F.Cu") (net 13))
 (via (at 153.25 111.25) (size 0.6) (drill 0.3) (layers "F.Cu" "B.Cu") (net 13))
 (via (at 153.25 92.75) (size 0.6) (drill 0.3) (layers "F.Cu" "B.Cu") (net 13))
 (segment (start 153.25 111.25) (end 153.25 92.75) (width 0.43) (layer "B.Cu") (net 13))
 (segment (start 97.23 117.25) (end 97.23 98.61) (width 0.23) (layer "F.Cu") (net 9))
 (segment (start 97.23 98.61) (end 111.615 84.225) (width 0.23) (layer "F.Cu") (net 9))
 (segment (start 149.51 83.24) (end 149.52 83.25) (width 0.23) (layer "F.Cu") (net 17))
 (segment (start 137.015 107.085) (end 140.415 107.085) (width 0.23) (layer "F.Cu") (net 17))
 (segment (start 140.415 107.085) (end 149.5 98) (width 0.23) (layer "F.Cu") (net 17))
 (segment (start 145.77 79.5) (end 149.51 83.24) (width 0.23) (layer "F.Cu") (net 17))
 (segment (start 149.5 98) (end 149.5 89.75) (width 0.23) (layer "F.Cu") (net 17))
 (via (at 149.5 89.75) (size 0.6) (drill 0.3) (layers "F.Cu" "B.Cu") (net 17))
 (via (at 149.51 83.24) (size 0.6) (drill 0.3) (layers "F.Cu" "B.Cu") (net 17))
 (segment (start 149.5 83.25) (end 149.5 89.75) (width 0.23) (layer "B.Cu") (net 17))
 (segment (start 149.51 83.24) (end 149.5 83.25) (width 0.23) (layer "B.Cu") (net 17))
 (segment (start 101.52 85) (end 101.52 91.23) (width 0.43) (layer "F.Cu") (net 18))
 (segment (start 107.5 96) (end 109 97.5) (width 0.43) (layer "F.Cu") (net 18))
 (segment (start 111.615 119.785) (end 110.035 119.785) (width 0.43) (layer "F.Cu") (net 18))
 (segment (start 109 97.5) (end 109 109) (width 0.43) (layer "F.Cu") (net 18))
 (segment (start 110.035 119.785) (end 109 118.75) (width 0.43) (layer "F.Cu") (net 18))
 (segment (start 101.52 91.23) (end 101.5 91.25) (width 0.43) (layer "F.Cu") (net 18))
 (via (at 101.5 91.25) (size 0.6) (drill 0.3) (layers "F.Cu" "B.Cu") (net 18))
 (via (at 109 109) (size 0.6) (drill 0.3) (layers "F.Cu" "B.Cu") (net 18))
 (via (at 109 118.75) (size 0.6) (drill 0.3) (layers "F.Cu" "B.Cu") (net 18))
 (via (at 107.5 96) (size 0.6) (drill 0.3) (layers "F.Cu" "B.Cu") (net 18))
 (segment (start 106.25 96) (end 107.5 96) (width 0.43) (layer "B.Cu") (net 18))
 (segment (start 101.5 91.25) (end 106.25 96) (width 0.43) (layer "B.Cu") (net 18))
 (segment (start 109 118.75) (end 109 109) (width 0.43) (layer "B.Cu") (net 18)))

